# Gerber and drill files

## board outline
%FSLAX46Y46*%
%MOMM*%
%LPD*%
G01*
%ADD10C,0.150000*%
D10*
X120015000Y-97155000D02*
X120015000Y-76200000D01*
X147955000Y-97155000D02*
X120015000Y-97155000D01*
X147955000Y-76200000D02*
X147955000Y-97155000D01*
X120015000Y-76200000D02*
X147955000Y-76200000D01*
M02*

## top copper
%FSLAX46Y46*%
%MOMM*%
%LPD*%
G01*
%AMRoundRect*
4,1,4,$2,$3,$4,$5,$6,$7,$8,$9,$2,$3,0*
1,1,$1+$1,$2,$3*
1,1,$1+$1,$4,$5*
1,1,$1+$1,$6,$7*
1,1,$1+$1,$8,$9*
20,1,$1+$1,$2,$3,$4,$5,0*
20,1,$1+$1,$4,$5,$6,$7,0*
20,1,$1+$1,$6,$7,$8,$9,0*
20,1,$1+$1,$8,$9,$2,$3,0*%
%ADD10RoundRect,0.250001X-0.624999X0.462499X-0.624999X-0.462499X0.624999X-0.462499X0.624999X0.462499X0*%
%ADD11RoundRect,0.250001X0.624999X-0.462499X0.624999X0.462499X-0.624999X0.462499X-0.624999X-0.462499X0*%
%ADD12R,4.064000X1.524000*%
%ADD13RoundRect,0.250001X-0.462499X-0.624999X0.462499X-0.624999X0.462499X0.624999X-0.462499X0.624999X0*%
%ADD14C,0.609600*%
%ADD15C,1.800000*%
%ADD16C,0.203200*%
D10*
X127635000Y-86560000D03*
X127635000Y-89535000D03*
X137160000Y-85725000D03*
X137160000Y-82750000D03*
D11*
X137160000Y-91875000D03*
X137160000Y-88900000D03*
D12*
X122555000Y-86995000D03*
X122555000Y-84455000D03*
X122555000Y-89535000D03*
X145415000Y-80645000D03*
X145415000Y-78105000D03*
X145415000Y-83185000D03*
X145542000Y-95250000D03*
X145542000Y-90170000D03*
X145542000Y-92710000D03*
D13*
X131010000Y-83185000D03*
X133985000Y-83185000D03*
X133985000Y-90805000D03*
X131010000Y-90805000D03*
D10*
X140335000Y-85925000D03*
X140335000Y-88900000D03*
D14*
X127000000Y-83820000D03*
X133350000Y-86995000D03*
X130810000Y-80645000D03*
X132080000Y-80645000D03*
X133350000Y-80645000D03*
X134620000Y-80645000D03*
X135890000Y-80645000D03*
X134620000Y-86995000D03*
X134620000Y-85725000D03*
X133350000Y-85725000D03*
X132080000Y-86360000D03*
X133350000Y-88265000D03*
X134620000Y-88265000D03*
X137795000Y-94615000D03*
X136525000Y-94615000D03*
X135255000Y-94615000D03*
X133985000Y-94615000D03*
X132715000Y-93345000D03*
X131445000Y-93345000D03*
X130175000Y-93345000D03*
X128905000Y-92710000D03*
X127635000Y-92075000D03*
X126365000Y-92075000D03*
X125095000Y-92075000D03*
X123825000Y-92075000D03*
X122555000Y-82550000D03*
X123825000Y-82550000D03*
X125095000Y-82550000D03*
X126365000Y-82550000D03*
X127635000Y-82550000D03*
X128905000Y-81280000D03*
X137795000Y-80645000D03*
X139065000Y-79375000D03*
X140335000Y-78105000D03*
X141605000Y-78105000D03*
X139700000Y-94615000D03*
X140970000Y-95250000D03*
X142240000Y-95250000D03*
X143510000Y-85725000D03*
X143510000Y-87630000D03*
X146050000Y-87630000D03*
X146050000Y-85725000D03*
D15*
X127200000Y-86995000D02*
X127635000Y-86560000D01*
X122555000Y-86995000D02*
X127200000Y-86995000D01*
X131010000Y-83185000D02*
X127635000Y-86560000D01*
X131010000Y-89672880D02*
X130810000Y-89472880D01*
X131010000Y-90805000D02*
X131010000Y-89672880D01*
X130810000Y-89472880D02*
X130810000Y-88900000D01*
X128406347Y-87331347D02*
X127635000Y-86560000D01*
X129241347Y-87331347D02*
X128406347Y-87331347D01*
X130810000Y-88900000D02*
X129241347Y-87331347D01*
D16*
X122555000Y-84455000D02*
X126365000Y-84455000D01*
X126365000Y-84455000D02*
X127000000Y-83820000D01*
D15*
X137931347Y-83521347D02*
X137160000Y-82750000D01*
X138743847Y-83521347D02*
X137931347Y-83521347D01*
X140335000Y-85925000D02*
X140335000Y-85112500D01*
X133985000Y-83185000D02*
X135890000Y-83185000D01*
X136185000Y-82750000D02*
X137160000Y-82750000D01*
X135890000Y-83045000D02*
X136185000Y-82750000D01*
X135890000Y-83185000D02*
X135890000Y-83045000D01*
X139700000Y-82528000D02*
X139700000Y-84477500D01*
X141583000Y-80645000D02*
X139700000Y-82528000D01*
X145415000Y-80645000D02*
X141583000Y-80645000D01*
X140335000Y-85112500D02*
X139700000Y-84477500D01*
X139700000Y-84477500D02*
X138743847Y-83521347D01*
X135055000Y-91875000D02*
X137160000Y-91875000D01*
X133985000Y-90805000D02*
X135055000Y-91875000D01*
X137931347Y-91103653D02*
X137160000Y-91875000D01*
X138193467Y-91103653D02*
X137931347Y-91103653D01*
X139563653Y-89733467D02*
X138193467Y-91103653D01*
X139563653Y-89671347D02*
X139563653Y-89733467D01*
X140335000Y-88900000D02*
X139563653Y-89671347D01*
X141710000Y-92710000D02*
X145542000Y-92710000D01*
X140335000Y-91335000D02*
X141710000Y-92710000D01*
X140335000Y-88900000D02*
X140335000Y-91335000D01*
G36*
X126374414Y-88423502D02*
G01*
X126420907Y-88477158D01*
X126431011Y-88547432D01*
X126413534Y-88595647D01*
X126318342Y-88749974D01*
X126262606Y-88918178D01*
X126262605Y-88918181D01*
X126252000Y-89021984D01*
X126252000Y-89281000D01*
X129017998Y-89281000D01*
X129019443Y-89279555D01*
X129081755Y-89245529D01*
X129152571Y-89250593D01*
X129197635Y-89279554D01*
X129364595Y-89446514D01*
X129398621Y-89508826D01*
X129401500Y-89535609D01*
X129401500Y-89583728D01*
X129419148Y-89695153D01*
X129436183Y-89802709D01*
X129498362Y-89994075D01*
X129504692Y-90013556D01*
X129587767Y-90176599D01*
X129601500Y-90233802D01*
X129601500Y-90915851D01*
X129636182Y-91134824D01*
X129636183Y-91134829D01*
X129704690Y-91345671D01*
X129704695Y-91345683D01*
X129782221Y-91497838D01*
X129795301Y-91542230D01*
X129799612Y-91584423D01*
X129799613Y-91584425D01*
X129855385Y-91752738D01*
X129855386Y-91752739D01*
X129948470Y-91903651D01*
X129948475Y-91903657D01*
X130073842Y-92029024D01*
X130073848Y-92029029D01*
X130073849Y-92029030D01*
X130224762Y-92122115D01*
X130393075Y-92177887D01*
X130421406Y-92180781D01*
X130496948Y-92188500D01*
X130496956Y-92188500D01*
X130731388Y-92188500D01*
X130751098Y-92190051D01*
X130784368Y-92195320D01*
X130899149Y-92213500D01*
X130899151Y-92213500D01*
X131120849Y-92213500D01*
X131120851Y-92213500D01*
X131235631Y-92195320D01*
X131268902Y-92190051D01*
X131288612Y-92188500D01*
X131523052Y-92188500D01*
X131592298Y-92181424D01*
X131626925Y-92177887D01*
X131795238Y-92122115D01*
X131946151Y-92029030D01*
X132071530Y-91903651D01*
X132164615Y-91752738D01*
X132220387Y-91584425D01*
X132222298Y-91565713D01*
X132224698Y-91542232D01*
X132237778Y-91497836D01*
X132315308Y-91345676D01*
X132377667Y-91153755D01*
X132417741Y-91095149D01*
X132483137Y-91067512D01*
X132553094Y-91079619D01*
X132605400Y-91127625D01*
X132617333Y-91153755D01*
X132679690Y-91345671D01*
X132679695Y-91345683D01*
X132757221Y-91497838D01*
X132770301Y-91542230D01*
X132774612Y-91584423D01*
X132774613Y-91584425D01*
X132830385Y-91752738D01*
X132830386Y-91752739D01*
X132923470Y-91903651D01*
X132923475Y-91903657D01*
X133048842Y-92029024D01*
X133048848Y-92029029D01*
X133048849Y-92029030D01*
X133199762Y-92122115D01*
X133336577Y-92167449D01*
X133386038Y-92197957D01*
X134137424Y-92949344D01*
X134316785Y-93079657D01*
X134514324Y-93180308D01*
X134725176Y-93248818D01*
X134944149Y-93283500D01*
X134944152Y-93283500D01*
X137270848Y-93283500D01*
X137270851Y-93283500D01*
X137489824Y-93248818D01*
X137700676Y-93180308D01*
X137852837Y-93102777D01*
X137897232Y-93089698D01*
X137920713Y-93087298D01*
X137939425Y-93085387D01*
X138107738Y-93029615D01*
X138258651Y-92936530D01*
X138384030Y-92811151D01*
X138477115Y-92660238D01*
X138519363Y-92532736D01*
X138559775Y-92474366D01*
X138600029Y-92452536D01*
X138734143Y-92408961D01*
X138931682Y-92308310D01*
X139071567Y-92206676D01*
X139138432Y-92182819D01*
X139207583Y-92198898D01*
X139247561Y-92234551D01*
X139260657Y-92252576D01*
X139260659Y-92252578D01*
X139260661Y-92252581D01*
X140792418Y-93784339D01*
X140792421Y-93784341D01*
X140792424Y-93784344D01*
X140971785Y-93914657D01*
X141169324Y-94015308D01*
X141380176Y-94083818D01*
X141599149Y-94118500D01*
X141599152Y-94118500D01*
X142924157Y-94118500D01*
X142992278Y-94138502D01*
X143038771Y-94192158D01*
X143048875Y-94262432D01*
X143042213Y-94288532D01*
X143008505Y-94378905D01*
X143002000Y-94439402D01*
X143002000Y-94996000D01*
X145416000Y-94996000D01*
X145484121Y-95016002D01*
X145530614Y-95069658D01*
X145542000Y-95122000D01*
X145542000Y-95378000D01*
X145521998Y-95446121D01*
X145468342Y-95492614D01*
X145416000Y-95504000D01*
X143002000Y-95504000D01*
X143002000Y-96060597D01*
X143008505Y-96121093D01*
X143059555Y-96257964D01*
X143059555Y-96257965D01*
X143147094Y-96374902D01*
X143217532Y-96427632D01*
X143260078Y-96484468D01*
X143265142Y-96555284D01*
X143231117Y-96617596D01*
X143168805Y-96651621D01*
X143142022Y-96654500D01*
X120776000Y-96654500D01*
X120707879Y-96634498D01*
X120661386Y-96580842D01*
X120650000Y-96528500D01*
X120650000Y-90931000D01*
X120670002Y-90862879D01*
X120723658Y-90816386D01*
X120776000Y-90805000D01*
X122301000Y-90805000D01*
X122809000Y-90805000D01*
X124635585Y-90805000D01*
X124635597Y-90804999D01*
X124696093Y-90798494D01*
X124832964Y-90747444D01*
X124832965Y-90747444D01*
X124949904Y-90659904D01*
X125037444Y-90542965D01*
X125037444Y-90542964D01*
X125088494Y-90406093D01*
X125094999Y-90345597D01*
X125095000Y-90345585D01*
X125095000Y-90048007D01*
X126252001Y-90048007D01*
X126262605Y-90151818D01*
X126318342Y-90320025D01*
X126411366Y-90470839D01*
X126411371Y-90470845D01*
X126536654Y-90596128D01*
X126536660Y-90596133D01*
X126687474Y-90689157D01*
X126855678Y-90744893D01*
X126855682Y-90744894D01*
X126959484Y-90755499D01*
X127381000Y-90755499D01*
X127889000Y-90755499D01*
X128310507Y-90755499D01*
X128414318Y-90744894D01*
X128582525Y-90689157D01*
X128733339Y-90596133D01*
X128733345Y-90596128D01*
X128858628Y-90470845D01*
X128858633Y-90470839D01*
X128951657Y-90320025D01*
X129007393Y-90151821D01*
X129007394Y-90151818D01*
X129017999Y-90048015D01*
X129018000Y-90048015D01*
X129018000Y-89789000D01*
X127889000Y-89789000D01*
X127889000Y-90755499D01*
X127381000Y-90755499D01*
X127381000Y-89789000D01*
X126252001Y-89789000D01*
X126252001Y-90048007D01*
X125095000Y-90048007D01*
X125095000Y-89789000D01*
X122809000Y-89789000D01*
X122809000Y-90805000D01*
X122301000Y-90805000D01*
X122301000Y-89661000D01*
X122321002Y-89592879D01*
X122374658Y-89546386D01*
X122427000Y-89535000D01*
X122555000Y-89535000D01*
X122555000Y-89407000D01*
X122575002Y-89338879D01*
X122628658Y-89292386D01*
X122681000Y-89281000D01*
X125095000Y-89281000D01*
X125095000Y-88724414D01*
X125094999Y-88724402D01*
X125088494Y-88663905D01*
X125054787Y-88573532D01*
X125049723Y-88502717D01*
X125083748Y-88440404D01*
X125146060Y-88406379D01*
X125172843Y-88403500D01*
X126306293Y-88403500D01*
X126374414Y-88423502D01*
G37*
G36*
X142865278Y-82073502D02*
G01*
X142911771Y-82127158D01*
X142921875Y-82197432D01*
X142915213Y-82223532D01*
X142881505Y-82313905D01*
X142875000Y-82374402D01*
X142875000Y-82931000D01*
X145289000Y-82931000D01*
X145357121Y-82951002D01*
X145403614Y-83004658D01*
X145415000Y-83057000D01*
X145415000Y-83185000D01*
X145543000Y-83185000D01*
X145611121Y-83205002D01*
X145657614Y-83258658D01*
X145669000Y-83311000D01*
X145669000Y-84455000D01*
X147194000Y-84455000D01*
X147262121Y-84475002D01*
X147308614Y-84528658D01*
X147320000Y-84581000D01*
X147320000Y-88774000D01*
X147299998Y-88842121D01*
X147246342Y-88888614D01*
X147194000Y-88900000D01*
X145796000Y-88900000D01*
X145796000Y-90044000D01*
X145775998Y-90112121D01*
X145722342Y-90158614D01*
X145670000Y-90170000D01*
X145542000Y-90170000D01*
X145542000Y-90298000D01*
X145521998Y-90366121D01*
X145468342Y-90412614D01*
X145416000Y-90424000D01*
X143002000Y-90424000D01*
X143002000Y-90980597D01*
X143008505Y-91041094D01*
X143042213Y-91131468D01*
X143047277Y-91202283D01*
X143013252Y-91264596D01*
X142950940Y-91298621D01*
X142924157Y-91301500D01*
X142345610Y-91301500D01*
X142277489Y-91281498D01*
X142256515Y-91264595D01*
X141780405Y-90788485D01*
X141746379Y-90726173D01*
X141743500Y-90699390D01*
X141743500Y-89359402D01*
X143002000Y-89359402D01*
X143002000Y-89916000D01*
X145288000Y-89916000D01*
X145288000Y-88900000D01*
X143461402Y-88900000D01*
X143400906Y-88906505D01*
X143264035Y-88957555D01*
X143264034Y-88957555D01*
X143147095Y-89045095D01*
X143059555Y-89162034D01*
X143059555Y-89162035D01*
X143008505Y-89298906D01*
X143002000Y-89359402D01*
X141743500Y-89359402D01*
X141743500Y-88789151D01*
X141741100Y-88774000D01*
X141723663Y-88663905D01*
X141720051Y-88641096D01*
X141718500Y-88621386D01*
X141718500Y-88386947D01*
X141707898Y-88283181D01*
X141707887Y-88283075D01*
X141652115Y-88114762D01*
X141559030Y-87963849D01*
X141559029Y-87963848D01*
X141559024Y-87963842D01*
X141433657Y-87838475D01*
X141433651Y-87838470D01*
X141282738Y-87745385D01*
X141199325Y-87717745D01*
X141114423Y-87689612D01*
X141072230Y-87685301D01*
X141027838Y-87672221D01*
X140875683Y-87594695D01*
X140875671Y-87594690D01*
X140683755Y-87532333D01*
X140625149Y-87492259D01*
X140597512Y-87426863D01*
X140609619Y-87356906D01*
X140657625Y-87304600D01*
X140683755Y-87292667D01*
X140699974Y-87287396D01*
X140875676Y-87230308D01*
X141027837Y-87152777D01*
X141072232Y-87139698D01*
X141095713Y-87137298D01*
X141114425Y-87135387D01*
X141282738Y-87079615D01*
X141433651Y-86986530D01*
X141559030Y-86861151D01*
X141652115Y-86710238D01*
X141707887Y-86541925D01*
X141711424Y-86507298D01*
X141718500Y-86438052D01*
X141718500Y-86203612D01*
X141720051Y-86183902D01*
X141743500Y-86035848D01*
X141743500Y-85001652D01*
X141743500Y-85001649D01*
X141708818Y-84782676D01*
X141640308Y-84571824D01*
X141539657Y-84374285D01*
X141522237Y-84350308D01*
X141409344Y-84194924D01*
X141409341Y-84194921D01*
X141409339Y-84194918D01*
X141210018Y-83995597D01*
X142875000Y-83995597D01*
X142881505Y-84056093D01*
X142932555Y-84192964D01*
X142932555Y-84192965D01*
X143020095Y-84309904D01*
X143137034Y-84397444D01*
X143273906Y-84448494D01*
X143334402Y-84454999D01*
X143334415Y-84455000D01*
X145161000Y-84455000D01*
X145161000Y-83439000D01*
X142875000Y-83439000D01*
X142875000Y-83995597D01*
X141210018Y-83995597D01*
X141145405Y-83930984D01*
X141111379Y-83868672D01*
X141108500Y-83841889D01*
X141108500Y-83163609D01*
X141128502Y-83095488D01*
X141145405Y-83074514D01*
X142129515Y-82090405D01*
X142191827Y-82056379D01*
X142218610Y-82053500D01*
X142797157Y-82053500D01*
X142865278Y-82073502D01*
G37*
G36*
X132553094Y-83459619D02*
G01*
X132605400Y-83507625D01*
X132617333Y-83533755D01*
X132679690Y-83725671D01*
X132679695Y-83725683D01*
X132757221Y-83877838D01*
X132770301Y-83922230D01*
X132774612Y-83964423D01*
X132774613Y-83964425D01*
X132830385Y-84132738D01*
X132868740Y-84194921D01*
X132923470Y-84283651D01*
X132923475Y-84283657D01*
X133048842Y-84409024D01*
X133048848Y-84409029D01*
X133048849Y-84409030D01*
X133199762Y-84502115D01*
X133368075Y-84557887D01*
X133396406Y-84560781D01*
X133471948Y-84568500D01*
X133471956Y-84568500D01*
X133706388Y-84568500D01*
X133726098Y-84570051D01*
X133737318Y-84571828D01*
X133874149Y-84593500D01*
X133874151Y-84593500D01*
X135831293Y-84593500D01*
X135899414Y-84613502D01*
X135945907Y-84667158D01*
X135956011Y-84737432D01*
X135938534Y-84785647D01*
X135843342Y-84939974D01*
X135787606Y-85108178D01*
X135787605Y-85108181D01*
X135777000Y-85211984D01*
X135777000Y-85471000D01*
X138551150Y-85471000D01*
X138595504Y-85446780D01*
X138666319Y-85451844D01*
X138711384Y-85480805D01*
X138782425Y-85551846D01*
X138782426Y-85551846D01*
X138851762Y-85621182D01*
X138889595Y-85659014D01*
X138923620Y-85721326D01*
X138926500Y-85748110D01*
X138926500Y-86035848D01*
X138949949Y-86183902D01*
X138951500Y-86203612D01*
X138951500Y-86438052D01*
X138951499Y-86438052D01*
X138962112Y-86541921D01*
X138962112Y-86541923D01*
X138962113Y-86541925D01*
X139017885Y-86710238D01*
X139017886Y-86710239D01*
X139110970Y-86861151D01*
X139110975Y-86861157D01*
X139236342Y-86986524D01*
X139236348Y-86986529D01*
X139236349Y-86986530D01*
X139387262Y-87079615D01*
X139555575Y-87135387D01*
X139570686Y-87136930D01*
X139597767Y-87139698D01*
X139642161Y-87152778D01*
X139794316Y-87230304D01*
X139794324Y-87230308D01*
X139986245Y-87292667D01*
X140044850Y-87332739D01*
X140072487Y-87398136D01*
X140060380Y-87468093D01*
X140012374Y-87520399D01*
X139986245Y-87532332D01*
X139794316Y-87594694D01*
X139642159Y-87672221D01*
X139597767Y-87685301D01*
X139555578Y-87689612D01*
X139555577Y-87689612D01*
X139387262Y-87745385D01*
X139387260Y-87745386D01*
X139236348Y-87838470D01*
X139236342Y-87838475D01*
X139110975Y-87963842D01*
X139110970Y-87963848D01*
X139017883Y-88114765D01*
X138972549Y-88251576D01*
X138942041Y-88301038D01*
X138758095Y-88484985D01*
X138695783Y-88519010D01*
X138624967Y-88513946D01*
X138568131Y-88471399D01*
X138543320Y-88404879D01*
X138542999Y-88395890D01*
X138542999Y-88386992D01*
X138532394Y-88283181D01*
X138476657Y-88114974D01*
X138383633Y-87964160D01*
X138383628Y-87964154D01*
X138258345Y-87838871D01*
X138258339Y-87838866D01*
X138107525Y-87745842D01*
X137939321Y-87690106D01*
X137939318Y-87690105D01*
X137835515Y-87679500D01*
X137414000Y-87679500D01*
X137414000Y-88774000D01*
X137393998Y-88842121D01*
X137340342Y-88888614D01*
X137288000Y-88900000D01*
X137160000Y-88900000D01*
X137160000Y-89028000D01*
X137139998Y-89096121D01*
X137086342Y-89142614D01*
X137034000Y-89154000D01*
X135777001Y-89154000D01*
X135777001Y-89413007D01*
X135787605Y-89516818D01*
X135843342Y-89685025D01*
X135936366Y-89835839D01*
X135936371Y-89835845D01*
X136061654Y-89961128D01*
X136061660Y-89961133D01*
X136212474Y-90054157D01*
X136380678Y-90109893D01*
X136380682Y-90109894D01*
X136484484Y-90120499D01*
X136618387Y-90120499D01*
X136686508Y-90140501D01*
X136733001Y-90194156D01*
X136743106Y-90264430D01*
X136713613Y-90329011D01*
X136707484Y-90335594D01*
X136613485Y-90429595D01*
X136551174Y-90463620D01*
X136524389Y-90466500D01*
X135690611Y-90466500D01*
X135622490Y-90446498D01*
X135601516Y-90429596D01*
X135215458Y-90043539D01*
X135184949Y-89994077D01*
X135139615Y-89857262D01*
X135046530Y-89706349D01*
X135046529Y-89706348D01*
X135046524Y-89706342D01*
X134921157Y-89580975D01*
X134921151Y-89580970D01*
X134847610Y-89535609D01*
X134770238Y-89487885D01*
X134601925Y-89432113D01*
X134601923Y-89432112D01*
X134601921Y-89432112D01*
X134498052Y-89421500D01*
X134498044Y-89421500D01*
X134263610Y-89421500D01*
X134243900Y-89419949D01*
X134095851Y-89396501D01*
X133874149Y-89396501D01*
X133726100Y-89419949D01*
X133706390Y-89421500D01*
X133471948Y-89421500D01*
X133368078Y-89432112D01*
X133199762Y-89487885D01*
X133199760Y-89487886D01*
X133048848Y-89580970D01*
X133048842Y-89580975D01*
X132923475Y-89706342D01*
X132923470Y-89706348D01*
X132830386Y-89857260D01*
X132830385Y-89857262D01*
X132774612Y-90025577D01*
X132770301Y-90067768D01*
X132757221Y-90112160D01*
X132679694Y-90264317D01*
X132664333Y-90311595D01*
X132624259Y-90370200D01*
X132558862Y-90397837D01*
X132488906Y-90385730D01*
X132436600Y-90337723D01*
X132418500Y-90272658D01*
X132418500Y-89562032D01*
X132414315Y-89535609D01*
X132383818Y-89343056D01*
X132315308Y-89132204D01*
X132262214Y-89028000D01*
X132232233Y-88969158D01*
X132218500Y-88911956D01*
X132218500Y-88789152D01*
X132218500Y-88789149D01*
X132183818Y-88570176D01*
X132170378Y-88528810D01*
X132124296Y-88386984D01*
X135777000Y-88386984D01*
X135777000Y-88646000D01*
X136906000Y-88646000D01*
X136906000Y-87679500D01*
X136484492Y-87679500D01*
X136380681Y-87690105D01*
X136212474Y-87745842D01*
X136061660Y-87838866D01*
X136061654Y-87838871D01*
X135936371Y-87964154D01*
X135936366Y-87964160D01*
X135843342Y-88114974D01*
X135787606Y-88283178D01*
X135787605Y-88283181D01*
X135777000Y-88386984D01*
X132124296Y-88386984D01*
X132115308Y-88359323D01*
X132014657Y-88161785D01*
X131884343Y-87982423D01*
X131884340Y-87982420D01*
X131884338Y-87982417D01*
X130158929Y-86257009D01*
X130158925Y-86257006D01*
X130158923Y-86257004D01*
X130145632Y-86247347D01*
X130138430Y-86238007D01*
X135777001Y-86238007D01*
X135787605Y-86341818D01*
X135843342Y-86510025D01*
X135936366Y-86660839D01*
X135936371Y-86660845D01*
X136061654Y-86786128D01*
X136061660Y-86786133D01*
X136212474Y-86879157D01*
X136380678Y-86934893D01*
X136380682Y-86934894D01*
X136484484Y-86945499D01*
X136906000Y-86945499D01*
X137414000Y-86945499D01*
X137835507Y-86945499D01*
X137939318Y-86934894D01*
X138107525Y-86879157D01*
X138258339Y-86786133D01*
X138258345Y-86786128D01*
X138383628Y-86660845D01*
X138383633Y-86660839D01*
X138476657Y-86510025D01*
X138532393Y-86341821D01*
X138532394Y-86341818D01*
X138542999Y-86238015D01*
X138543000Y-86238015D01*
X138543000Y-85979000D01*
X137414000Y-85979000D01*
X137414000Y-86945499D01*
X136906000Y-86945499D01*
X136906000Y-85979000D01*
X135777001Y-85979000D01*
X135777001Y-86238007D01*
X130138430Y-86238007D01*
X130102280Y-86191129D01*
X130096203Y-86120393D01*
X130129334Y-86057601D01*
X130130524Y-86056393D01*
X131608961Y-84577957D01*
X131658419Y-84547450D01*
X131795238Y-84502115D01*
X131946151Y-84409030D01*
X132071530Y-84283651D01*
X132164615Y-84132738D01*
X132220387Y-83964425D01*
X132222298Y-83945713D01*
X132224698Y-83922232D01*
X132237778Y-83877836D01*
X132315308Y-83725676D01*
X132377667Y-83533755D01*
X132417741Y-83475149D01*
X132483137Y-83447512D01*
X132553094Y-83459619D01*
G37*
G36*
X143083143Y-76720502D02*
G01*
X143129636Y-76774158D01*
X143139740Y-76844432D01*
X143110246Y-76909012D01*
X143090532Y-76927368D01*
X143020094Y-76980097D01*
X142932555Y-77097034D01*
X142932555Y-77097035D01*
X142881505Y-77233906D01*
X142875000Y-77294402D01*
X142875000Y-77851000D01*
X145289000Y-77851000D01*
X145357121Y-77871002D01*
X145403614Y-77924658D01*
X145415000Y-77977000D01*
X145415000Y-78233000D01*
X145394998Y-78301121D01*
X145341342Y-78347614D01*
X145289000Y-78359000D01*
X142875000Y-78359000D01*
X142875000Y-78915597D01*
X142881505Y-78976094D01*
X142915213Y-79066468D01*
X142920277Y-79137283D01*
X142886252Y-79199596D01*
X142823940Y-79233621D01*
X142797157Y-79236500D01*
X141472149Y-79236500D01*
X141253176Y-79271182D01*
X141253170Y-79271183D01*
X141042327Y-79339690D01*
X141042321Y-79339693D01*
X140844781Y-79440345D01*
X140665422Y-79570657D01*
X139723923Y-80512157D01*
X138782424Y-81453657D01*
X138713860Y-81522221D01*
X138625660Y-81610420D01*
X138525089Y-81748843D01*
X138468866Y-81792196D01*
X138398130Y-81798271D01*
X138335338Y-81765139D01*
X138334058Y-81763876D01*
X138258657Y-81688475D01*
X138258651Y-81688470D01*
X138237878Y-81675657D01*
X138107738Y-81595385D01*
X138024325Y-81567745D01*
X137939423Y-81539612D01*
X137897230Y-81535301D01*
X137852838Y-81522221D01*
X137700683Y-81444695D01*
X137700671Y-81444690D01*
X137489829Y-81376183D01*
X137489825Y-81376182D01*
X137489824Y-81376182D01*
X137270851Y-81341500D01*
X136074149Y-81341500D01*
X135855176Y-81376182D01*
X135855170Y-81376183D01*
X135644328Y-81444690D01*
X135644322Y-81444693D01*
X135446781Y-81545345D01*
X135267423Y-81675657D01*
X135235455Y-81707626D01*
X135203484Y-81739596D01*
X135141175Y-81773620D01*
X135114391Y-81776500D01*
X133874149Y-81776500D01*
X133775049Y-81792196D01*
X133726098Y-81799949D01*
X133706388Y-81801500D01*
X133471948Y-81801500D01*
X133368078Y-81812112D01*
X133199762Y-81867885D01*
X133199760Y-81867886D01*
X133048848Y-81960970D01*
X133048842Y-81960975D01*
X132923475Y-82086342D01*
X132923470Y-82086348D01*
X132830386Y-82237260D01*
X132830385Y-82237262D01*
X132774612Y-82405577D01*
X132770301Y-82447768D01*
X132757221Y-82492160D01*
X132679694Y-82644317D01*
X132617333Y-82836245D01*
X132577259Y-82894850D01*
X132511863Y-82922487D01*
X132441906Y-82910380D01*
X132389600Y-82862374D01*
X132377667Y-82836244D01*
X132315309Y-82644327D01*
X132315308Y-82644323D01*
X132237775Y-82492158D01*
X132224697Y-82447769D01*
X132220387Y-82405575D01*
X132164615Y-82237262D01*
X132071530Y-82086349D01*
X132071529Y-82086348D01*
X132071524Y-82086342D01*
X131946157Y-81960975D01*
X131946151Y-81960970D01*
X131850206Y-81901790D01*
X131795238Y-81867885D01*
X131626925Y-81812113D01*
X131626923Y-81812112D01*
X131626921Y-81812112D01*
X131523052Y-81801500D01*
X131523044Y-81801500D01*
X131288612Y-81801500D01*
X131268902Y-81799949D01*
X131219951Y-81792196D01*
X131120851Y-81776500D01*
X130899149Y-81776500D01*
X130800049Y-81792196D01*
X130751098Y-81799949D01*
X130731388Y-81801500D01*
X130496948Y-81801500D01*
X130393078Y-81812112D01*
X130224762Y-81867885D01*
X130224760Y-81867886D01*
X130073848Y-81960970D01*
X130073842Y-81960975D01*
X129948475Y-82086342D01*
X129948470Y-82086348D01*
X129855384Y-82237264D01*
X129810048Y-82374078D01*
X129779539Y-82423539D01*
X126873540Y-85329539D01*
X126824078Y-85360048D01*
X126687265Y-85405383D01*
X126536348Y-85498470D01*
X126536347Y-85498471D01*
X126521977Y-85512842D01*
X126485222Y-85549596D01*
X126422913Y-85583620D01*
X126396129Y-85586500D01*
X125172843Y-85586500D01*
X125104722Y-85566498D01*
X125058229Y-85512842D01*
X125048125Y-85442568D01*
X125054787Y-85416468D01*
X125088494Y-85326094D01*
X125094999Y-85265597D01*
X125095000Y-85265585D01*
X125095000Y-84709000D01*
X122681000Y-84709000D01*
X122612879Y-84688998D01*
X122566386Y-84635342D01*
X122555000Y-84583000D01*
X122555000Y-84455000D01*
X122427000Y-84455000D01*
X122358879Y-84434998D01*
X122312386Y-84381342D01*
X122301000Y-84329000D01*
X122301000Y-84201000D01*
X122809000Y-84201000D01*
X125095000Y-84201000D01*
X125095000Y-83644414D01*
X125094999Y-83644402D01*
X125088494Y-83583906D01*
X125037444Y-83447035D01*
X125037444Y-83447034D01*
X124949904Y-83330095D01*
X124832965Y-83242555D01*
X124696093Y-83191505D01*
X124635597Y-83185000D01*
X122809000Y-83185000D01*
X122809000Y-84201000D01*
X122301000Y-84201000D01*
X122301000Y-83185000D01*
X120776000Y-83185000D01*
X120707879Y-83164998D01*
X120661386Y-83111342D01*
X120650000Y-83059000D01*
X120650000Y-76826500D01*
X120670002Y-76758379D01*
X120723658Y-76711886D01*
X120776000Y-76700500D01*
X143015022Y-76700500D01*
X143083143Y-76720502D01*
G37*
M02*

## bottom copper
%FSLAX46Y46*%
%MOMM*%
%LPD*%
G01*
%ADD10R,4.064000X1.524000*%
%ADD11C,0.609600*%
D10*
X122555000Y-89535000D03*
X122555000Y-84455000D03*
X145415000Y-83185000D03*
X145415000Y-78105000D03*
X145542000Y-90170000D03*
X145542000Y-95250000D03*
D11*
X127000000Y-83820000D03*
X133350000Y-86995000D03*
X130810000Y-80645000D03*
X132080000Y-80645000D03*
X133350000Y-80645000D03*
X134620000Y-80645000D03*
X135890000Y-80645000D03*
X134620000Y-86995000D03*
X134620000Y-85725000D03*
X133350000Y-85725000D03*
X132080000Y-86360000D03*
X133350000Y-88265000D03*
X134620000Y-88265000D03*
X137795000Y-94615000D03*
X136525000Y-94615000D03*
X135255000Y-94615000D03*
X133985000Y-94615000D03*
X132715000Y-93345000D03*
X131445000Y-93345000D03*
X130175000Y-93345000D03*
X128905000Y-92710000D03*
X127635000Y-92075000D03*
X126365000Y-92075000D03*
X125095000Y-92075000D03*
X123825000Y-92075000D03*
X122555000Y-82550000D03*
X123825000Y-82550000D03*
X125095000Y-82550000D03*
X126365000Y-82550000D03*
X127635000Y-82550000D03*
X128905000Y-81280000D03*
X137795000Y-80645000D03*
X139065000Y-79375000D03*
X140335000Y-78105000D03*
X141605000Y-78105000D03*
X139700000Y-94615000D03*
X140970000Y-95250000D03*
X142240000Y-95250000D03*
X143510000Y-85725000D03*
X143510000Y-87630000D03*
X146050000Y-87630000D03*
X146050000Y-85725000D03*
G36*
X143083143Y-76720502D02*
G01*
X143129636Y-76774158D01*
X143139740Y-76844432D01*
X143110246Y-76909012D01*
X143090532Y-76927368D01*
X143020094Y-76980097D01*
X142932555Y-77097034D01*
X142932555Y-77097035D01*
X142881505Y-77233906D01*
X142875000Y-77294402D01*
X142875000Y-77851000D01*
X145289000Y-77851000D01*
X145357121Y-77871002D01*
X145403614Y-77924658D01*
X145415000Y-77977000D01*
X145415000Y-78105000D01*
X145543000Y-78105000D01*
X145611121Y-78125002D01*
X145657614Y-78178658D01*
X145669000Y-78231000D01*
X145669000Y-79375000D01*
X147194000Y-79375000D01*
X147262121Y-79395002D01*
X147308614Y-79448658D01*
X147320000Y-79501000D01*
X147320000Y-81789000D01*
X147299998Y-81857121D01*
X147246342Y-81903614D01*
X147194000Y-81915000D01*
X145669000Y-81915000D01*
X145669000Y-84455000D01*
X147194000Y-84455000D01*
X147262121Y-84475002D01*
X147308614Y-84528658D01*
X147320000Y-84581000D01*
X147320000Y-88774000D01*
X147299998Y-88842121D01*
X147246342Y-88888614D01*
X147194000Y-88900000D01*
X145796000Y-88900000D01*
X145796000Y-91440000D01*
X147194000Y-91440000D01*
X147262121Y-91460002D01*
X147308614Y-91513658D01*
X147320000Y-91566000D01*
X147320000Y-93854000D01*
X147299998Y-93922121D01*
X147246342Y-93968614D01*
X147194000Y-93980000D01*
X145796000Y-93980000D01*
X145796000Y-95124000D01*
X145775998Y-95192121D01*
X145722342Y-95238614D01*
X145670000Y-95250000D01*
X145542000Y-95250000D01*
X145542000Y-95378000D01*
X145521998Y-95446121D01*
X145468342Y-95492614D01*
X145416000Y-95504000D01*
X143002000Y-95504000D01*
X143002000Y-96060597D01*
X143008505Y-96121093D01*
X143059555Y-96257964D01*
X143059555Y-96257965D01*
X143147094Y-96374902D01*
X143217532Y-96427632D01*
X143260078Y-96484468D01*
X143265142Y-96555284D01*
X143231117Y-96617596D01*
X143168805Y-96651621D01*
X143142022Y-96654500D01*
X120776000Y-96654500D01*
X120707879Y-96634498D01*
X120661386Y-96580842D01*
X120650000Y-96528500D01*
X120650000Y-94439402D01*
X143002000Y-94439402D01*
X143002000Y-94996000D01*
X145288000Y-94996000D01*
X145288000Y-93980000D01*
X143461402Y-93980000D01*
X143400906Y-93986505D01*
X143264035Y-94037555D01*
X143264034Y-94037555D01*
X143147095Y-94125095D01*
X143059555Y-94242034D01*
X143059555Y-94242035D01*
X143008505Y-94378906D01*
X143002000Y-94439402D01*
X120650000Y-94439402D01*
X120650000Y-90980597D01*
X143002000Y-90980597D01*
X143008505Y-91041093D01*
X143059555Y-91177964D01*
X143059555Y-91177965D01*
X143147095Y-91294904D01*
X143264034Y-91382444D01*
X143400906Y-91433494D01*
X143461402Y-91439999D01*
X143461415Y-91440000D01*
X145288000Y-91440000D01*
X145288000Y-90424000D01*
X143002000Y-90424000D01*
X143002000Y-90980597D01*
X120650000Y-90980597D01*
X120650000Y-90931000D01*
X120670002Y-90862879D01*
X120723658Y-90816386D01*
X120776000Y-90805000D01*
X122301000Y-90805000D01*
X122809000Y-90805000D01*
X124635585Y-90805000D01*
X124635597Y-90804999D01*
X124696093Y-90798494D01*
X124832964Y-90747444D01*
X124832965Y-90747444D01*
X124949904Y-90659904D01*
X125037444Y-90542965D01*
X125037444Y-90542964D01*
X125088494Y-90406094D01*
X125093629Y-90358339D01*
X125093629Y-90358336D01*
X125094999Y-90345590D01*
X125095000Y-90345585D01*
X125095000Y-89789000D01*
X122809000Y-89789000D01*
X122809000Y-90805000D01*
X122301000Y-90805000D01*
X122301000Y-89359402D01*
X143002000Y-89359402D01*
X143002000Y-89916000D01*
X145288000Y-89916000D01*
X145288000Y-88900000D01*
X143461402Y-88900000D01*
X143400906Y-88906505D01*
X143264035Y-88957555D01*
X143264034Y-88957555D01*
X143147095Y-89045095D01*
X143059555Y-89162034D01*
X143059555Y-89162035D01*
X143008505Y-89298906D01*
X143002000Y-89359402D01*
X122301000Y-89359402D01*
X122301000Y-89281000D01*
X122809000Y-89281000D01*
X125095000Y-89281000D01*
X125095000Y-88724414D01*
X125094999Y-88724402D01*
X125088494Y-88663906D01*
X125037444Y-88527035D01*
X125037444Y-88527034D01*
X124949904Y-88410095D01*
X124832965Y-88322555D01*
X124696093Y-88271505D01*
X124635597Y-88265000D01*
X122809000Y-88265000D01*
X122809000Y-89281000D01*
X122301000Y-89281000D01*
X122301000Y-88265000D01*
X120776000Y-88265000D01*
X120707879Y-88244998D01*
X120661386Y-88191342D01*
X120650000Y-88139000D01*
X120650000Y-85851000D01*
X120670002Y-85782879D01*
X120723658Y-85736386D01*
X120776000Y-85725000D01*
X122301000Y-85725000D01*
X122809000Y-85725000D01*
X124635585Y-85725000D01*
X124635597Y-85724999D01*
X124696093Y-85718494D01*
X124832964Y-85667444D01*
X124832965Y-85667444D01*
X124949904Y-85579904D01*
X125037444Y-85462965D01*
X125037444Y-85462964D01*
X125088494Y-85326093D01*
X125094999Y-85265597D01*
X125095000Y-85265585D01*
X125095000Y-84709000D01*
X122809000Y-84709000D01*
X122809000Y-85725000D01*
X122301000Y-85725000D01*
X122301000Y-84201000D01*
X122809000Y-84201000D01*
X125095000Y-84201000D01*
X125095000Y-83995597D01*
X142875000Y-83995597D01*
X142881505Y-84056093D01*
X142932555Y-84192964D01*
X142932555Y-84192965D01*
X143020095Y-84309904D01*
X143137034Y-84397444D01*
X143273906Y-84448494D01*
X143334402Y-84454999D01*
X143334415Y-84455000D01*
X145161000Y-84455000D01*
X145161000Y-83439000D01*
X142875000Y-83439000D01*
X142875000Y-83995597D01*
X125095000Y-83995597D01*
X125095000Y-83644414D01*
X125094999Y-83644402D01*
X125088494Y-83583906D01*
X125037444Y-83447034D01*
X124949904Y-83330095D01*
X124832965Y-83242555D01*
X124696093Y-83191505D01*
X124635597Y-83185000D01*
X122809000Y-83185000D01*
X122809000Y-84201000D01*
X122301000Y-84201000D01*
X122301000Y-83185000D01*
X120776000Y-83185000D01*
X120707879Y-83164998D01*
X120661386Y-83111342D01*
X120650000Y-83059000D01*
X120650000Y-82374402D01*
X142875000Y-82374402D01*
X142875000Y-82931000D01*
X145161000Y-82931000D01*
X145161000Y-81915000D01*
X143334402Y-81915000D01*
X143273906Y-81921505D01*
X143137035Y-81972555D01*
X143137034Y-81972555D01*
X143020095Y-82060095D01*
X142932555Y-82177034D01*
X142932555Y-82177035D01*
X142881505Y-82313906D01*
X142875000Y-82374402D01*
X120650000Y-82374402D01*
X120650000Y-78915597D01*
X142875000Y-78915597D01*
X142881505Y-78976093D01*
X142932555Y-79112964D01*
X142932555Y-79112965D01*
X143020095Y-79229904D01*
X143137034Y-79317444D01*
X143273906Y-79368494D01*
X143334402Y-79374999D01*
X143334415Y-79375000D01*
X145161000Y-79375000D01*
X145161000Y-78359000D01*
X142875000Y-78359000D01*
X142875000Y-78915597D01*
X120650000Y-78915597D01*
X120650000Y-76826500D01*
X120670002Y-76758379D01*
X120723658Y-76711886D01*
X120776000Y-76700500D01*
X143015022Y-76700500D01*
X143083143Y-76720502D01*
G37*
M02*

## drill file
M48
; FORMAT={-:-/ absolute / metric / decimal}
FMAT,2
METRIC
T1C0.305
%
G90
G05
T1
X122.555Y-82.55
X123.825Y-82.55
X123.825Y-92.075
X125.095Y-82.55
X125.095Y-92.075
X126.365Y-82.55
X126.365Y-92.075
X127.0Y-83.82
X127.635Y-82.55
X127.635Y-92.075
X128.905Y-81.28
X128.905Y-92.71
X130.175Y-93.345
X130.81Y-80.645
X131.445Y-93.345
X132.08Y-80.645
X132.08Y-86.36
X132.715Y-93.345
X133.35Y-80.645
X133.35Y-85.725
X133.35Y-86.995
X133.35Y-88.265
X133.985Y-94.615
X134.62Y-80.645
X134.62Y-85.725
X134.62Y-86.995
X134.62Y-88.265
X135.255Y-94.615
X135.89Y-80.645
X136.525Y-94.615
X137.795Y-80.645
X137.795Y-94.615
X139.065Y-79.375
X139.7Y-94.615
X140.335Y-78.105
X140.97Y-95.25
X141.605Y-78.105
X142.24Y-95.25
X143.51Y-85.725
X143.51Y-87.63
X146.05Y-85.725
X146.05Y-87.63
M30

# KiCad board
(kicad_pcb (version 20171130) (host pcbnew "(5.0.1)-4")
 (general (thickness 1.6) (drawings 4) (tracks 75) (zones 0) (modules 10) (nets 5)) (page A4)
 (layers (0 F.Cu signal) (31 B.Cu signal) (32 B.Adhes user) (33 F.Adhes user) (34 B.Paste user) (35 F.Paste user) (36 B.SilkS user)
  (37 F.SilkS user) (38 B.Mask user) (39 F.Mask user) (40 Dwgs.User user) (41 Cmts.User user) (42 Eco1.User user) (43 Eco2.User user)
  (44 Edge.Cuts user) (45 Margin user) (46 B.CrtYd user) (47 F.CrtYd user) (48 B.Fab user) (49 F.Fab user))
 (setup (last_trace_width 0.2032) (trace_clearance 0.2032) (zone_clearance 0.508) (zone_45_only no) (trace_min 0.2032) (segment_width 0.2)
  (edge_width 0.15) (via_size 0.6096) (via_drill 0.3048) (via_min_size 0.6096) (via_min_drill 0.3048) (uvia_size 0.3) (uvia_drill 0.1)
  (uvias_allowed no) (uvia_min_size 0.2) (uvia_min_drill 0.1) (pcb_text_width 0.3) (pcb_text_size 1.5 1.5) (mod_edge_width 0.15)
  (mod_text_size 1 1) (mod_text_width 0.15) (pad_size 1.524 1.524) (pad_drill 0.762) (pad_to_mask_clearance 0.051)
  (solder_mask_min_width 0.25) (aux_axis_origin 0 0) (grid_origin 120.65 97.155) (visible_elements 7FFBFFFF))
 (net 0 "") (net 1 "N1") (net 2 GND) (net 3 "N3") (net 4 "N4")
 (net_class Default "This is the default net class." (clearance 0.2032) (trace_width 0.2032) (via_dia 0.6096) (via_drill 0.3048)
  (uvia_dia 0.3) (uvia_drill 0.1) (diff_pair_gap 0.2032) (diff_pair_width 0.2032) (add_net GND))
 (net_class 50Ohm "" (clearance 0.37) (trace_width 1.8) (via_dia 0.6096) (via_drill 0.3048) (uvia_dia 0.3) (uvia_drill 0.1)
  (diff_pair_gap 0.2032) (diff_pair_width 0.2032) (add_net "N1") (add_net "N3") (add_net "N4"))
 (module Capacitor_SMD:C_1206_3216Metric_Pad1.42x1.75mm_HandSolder (layer F.Cu) (at 127.635 88.0475 270)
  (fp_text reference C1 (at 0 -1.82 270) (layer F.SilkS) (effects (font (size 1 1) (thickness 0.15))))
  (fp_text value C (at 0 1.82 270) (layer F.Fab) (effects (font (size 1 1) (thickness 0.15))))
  (pad 1 smd roundrect (at -1.4875 0 270) (size 1.425 1.75) (layers F.Cu F.Paste F.Mask) (roundrect_rratio 0.175439) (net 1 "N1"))
  (pad 2 smd roundrect (at 1.4875 0 270) (size 1.425 1.75) (layers F.Cu F.Paste F.Mask) (roundrect_rratio 0.175439) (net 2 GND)))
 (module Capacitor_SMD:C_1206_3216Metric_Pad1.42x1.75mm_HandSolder (layer F.Cu) (at 137.16 84.2375 270)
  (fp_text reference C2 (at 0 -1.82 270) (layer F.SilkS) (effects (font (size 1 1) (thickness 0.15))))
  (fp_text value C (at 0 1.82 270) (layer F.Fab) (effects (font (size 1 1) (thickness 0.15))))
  (pad 2 smd roundrect (at 1.4875 0 270) (size 1.425 1.75) (layers F.Cu F.Paste F.Mask) (roundrect_rratio 0.175439) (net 2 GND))
  (pad 1 smd roundrect (at -1.4875 0 270) (size 1.425 1.75) (layers F.Cu F.Paste F.Mask) (roundrect_rratio 0.175439) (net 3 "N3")))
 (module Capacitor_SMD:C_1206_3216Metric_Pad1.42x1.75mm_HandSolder (layer F.Cu) (at 137.16 90.3875 90)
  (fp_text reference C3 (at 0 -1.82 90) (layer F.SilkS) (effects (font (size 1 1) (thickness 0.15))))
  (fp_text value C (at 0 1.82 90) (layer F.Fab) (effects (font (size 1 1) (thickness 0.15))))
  (pad 1 smd roundrect (at -1.4875 0 90) (size 1.425 1.75) (layers F.Cu F.Paste F.Mask) (roundrect_rratio 0.175439) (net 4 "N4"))
  (pad 2 smd roundrect (at 1.4875 0 90) (size 1.425 1.75) (layers F.Cu F.Paste F.Mask) (roundrect_rratio 0.175439) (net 2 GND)))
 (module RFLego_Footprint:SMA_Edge (layer F.Cu) (at 120.523 86.995)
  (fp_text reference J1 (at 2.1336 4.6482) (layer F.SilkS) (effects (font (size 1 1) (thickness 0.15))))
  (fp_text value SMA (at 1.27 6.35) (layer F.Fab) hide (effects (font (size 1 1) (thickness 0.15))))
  (pad 1 smd rect (at 2.032 0) (size 4.064 1.524) (layers F.Cu F.Mask) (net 1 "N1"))
  (pad 2 smd rect (at 2.032 -2.54) (size 4.064 1.524) (layers F.Cu F.Mask) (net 2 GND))
  (pad 2 smd rect (at 2.032 2.54) (size 4.064 1.524) (layers B.Cu B.Mask) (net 2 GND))
  (pad 2 smd rect (at 2.032 -2.54) (size 4.064 1.524) (layers B.Cu B.Mask) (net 2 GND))
  (pad 2 smd rect (at 2.032 2.54) (size 4.064 1.524) (layers F.Cu F.Mask) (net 2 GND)))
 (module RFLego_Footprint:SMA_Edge (layer F.Cu) (at 143.383 80.645)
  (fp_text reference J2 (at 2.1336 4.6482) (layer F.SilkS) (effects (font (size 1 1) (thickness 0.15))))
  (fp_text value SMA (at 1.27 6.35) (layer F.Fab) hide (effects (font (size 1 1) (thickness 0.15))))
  (pad 1 smd rect (at 2.032 0) (size 4.064 1.524) (layers F.Cu F.Mask) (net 3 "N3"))
  (pad 2 smd rect (at 2.032 -2.54) (size 4.064 1.524) (layers F.Cu F.Mask) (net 2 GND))
  (pad 2 smd rect (at 2.032 2.54) (size 4.064 1.524) (layers B.Cu B.Mask) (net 2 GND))
  (pad 2 smd rect (at 2.032 -2.54) (size 4.064 1.524) (layers B.Cu B.Mask) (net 2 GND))
  (pad 2 smd rect (at 2.032 2.54) (size 4.064 1.524) (layers F.Cu F.Mask) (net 2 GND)))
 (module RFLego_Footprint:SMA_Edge (layer F.Cu) (at 143.51 92.71)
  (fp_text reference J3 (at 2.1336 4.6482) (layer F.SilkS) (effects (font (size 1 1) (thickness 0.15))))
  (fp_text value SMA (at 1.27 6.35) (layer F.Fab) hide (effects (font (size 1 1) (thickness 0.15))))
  (pad 2 smd rect (at 2.032 2.54) (size 4.064 1.524) (layers F.Cu F.Mask) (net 2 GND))
  (pad 2 smd rect (at 2.032 -2.54) (size 4.064 1.524) (layers B.Cu B.Mask) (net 2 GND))
  (pad 2 smd rect (at 2.032 2.54) (size 4.064 1.524) (layers B.Cu B.Mask) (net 2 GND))
  (pad 2 smd rect (at 2.032 -2.54) (size 4.064 1.524) (layers F.Cu F.Mask) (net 2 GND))
  (pad 1 smd rect (at 2.032 0) (size 4.064 1.524) (layers F.Cu F.Mask) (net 4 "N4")))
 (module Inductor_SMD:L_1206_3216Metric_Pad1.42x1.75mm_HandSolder (layer F.Cu) (at 132.4975 83.185)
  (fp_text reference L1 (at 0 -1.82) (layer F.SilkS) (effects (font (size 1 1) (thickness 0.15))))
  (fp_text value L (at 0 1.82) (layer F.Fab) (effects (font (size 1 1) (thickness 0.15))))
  (pad 1 smd roundrect (at -1.4875 0) (size 1.425 1.75) (layers F.Cu F.Paste F.Mask) (roundrect_rratio 0.175439) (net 1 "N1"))
  (pad 2 smd roundrect (at 1.4875 0) (size 1.425 1.75) (layers F.Cu F.Paste F.Mask) (roundrect_rratio 0.175439) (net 3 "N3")))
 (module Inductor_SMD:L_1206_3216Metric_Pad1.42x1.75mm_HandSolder (layer F.Cu) (at 132.4975 90.805)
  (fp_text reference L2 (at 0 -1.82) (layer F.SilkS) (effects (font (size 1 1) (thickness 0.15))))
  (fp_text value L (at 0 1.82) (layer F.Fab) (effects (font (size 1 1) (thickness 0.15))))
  (pad 2 smd roundrect (at 1.4875 0) (size 1.425 1.75) (layers F.Cu F.Paste F.Mask) (roundrect_rratio 0.175439) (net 4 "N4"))
  (pad 1 smd roundrect (at -1.4875 0) (size 1.425 1.75) (layers F.Cu F.Paste F.Mask) (roundrect_rratio 0.175439) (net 1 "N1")))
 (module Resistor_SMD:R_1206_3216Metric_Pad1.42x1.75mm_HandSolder (layer F.Cu) (at 140.335 87.4125 270)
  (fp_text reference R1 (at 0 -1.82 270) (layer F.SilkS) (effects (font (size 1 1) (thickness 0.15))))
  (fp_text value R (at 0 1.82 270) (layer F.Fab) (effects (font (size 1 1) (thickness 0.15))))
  (pad 1 smd roundrect (at -1.4875 0 270) (size 1.425 1.75) (layers F.Cu F.Paste F.Mask) (roundrect_rratio 0.175439) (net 3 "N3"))
  (pad 2 smd roundrect (at 1.4875 0 270) (size 1.425 1.75) (layers F.Cu F.Paste F.Mask) (roundrect_rratio 0.175439) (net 4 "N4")))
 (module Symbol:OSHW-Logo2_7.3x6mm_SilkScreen (layer F.Cu) (at 125.095 79.375)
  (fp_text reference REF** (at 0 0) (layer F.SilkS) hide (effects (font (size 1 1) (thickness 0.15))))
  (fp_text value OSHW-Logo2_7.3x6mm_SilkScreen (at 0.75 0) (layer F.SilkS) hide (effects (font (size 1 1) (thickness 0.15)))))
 (gr_line (start 120.015 97.155) (end 120.015 76.2) (layer Edge.Cuts) (width 0.15))
 (gr_line (start 147.955 97.155) (end 120.015 97.155) (layer Edge.Cuts) (width 0.15))
 (gr_line (start 147.955 76.2) (end 147.955 97.155) (layer Edge.Cuts) (width 0.15))
 (gr_line (start 120.015 76.2) (end 147.955 76.2) (layer Edge.Cuts) (width 0.15))
 (segment (start 127.2 86.995) (end 127.635 86.56) (width 1.8) (layer F.Cu) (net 1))
 (segment (start 122.555 86.995) (end 127.2 86.995) (width 1.8) (layer F.Cu) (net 1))
 (segment (start 131.01 83.185) (end 127.635 86.56) (width 1.8) (layer F.Cu) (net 1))
 (segment (start 131.01 89.67288) (end 130.81 89.47288) (width 1.8) (layer F.Cu) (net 1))
 (segment (start 131.01 90.805) (end 131.01 89.67288) (width 1.8) (layer F.Cu) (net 1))
 (segment (start 130.81 89.47288) (end 130.81 88.9) (width 1.8) (layer F.Cu) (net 1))
 (segment (start 128.406347 87.331347) (end 127.635 86.56) (width 1.8) (layer F.Cu) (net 1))
 (segment (start 129.241347 87.331347) (end 128.406347 87.331347) (width 1.8) (layer F.Cu) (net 1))
 (segment (start 130.81 88.9) (end 129.241347 87.331347) (width 1.8) (layer F.Cu) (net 1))
 (via (at 127 83.82) (size 0.6096) (drill 0.3048) (layers F.Cu B.Cu) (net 2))
 (segment (start 122.555 84.455) (end 126.365 84.455) (width 0.2032) (layer F.Cu) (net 2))
 (segment (start 126.365 84.455) (end 127 83.82) (width 0.2032) (layer F.Cu) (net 2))
 (via (at 133.35 86.995) (size 0.6096) (drill 0.3048) (layers F.Cu B.Cu) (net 2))
 (via (at 130.81 80.645) (size 0.6096) (drill 0.3048) (layers F.Cu B.Cu) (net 2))
 (via (at 132.08 80.645) (size 0.6096) (drill 0.3048) (layers F.Cu B.Cu) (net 2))
 (via (at 133.35 80.645) (size 0.6096) (drill 0.3048) (layers F.Cu B.Cu) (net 2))
 (via (at 134.62 80.645) (size 0.6096) (drill 0.3048) (layers F.Cu B.Cu) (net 2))
 (via (at 135.89 80.645) (size 0.6096) (drill 0.3048) (layers F.Cu B.Cu) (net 2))
 (via (at 134.62 86.995) (size 0.6096) (drill 0.3048) (layers F.Cu B.Cu) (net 2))
 (via (at 134.62 85.725) (size 0.6096) (drill 0.3048) (layers F.Cu B.Cu) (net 2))
 (via (at 133.35 85.725) (size 0.6096) (drill 0.3048) (layers F.Cu B.Cu) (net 2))
 (via (at 132.08 86.36) (size 0.6096) (drill 0.3048) (layers F.Cu B.Cu) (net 2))
 (via (at 133.35 88.265) (size 0.6096) (drill 0.3048) (layers F.Cu B.Cu) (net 2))
 (via (at 134.62 88.265) (size 0.6096) (drill 0.3048) (layers F.Cu B.Cu) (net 2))
 (via (at 137.795 94.615) (size 0.6096) (drill 0.3048) (layers F.Cu B.Cu) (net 2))
 (via (at 136.525 94.615) (size 0.6096) (drill 0.3048) (layers F.Cu B.Cu) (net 2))
 (via (at 135.255 94.615) (size 0.6096) (drill 0.3048) (layers F.Cu B.Cu) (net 2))
 (via (at 133.985 94.615) (size 0.6096) (drill 0.3048) (layers F.Cu B.Cu) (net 2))
 (via (at 132.715 93.345) (size 0.6096) (drill 0.3048) (layers F.Cu B.Cu) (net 2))
 (via (at 131.445 93.345) (size 0.6096) (drill 0.3048) (layers F.Cu B.Cu) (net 2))
 (via (at 130.175 93.345) (size 0.6096) (drill 0.3048) (layers F.Cu B.Cu) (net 2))
 (via (at 128.905 92.71) (size 0.6096) (drill 0.3048) (layers F.Cu B.Cu) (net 2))
 (via (at 127.635 92.075) (size 0.6096) (drill 0.3048) (layers F.Cu B.Cu) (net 2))
 (via (at 126.365 92.075) (size 0.6096) (drill 0.3048) (layers F.Cu B.Cu) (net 2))
 (via (at 125.095 92.075) (size 0.6096) (drill 0.3048) (layers F.Cu B.Cu) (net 2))
 (via (at 123.825 92.075) (size 0.6096) (drill 0.3048) (layers F.Cu B.Cu) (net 2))
 (via (at 122.555 82.55) (size 0.6096) (drill 0.3048) (layers F.Cu B.Cu) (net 2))
 (via (at 123.825 82.55) (size 0.6096) (drill 0.3048) (layers F.Cu B.Cu) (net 2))
 (via (at 125.095 82.55) (size 0.6096) (drill 0.3048) (layers F.Cu B.Cu) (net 2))
 (via (at 126.365 82.55) (size 0.6096) (drill 0.3048) (layers F.Cu B.Cu) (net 2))
 (via (at 127.635 82.55) (size 0.6096) (drill 0.3048) (layers F.Cu B.Cu) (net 2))
 (via (at 128.905 81.28) (size 0.6096) (drill 0.3048) (layers F.Cu B.Cu) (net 2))
 (via (at 137.795 80.645) (size 0.6096) (drill 0.3048) (layers F.Cu B.Cu) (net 2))
 (via (at 139.065 79.375) (size 0.6096) (drill 0.3048) (layers F.Cu B.Cu) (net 2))
 (via (at 140.335 78.105) (size 0.6096) (drill 0.3048) (layers F.Cu B.Cu) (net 2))
 (via (at 141.605 78.105) (size 0.6096) (drill 0.3048) (layers F.Cu B.Cu) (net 2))
 (via (at 139.7 94.615) (size 0.6096) (drill 0.3048) (layers F.Cu B.Cu) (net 2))
 (via (at 140.97 95.25) (size 0.6096) (drill 0.3048) (layers F.Cu B.Cu) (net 2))
 (via (at 142.24 95.25) (size 0.6096) (drill 0.3048) (layers F.Cu B.Cu) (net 2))
 (via (at 143.51 85.725) (size 0.6096) (drill 0.3048) (layers F.Cu B.Cu) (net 2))
 (via (at 143.51 87.63) (size 0.6096) (drill 0.3048) (layers F.Cu B.Cu) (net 2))
 (via (at 146.05 87.63) (size 0.6096) (drill 0.3048) (layers F.Cu B.Cu) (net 2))
 (via (at 146.05 85.725) (size 0.6096) (drill 0.3048) (layers F.Cu B.Cu) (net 2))
 (segment (start 137.931347 83.521347) (end 137.16 82.75) (width 1.8) (layer F.Cu) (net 3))
 (segment (start 138.743847 83.521347) (end 137.931347 83.521347) (width 1.8) (layer F.Cu) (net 3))
 (segment (start 140.335 85.925) (end 140.335 85.1125) (width 1.8) (layer F.Cu) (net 3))
 (segment (start 133.985 83.185) (end 135.89 83.185) (width 1.8) (layer F.Cu) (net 3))
 (segment (start 136.185 82.75) (end 137.16 82.75) (width 1.8) (layer F.Cu) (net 3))
 (segment (start 135.89 83.045) (end 136.185 82.75) (width 1.8) (layer F.Cu) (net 3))
 (segment (start 135.89 83.185) (end 135.89 83.045) (width 1.8) (layer F.Cu) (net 3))
 (segment (start 139.7 82.528) (end 139.7 84.4775) (width 1.8) (layer F.Cu) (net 3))
 (segment (start 141.583 80.645) (end 139.7 82.528) (width 1.8) (layer F.Cu) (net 3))
 (segment (start 145.415 80.645) (end 141.583 80.645) (width 1.8) (layer F.Cu) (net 3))
 (segment (start 140.335 85.1125) (end 139.7 84.4775) (width 1.8) (layer F.Cu) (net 3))
 (segment (start 139.7 84.4775) (end 138.743847 83.521347) (width 1.8) (layer F.Cu) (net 3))
 (segment (start 135.055 91.875) (end 137.16 91.875) (width 1.8) (layer F.Cu) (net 4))
 (segment (start 133.985 90.805) (end 135.055 91.875) (width 1.8) (layer F.Cu) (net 4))
 (segment (start 137.931347 91.103653) (end 137.16 91.875) (width 1.8) (layer F.Cu) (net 4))
 (segment (start 138.193467 91.103653) (end 137.931347 91.103653) (width 1.8) (layer F.Cu) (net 4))
 (segment (start 139.563653 89.733467) (end 138.193467 91.103653) (width 1.8) (layer F.Cu) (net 4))
 (segment (start 139.563653 89.671347) (end 139.563653 89.733467) (width 1.8) (layer F.Cu) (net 4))
 (segment (start 140.335 88.9) (end 139.563653 89.671347) (width 1.8) (layer F.Cu) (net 4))
 (segment (start 141.71 92.71) (end 145.542 92.71) (width 1.8) (layer F.Cu) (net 4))
 (segment (start 140.335 91.335) (end 141.71 92.71) (width 1.8) (layer F.Cu) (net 4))
 (segment (start 140.335 88.9) (end 140.335 91.335) (width 1.8) (layer F.Cu) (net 4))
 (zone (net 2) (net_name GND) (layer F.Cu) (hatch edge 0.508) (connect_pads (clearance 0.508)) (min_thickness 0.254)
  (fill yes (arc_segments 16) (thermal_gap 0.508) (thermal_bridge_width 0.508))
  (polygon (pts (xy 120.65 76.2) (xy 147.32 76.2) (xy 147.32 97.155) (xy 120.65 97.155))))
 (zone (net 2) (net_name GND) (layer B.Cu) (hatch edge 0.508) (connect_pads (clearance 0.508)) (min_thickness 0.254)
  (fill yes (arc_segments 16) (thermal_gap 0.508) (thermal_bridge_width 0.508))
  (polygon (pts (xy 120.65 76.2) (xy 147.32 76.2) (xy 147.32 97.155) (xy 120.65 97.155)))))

